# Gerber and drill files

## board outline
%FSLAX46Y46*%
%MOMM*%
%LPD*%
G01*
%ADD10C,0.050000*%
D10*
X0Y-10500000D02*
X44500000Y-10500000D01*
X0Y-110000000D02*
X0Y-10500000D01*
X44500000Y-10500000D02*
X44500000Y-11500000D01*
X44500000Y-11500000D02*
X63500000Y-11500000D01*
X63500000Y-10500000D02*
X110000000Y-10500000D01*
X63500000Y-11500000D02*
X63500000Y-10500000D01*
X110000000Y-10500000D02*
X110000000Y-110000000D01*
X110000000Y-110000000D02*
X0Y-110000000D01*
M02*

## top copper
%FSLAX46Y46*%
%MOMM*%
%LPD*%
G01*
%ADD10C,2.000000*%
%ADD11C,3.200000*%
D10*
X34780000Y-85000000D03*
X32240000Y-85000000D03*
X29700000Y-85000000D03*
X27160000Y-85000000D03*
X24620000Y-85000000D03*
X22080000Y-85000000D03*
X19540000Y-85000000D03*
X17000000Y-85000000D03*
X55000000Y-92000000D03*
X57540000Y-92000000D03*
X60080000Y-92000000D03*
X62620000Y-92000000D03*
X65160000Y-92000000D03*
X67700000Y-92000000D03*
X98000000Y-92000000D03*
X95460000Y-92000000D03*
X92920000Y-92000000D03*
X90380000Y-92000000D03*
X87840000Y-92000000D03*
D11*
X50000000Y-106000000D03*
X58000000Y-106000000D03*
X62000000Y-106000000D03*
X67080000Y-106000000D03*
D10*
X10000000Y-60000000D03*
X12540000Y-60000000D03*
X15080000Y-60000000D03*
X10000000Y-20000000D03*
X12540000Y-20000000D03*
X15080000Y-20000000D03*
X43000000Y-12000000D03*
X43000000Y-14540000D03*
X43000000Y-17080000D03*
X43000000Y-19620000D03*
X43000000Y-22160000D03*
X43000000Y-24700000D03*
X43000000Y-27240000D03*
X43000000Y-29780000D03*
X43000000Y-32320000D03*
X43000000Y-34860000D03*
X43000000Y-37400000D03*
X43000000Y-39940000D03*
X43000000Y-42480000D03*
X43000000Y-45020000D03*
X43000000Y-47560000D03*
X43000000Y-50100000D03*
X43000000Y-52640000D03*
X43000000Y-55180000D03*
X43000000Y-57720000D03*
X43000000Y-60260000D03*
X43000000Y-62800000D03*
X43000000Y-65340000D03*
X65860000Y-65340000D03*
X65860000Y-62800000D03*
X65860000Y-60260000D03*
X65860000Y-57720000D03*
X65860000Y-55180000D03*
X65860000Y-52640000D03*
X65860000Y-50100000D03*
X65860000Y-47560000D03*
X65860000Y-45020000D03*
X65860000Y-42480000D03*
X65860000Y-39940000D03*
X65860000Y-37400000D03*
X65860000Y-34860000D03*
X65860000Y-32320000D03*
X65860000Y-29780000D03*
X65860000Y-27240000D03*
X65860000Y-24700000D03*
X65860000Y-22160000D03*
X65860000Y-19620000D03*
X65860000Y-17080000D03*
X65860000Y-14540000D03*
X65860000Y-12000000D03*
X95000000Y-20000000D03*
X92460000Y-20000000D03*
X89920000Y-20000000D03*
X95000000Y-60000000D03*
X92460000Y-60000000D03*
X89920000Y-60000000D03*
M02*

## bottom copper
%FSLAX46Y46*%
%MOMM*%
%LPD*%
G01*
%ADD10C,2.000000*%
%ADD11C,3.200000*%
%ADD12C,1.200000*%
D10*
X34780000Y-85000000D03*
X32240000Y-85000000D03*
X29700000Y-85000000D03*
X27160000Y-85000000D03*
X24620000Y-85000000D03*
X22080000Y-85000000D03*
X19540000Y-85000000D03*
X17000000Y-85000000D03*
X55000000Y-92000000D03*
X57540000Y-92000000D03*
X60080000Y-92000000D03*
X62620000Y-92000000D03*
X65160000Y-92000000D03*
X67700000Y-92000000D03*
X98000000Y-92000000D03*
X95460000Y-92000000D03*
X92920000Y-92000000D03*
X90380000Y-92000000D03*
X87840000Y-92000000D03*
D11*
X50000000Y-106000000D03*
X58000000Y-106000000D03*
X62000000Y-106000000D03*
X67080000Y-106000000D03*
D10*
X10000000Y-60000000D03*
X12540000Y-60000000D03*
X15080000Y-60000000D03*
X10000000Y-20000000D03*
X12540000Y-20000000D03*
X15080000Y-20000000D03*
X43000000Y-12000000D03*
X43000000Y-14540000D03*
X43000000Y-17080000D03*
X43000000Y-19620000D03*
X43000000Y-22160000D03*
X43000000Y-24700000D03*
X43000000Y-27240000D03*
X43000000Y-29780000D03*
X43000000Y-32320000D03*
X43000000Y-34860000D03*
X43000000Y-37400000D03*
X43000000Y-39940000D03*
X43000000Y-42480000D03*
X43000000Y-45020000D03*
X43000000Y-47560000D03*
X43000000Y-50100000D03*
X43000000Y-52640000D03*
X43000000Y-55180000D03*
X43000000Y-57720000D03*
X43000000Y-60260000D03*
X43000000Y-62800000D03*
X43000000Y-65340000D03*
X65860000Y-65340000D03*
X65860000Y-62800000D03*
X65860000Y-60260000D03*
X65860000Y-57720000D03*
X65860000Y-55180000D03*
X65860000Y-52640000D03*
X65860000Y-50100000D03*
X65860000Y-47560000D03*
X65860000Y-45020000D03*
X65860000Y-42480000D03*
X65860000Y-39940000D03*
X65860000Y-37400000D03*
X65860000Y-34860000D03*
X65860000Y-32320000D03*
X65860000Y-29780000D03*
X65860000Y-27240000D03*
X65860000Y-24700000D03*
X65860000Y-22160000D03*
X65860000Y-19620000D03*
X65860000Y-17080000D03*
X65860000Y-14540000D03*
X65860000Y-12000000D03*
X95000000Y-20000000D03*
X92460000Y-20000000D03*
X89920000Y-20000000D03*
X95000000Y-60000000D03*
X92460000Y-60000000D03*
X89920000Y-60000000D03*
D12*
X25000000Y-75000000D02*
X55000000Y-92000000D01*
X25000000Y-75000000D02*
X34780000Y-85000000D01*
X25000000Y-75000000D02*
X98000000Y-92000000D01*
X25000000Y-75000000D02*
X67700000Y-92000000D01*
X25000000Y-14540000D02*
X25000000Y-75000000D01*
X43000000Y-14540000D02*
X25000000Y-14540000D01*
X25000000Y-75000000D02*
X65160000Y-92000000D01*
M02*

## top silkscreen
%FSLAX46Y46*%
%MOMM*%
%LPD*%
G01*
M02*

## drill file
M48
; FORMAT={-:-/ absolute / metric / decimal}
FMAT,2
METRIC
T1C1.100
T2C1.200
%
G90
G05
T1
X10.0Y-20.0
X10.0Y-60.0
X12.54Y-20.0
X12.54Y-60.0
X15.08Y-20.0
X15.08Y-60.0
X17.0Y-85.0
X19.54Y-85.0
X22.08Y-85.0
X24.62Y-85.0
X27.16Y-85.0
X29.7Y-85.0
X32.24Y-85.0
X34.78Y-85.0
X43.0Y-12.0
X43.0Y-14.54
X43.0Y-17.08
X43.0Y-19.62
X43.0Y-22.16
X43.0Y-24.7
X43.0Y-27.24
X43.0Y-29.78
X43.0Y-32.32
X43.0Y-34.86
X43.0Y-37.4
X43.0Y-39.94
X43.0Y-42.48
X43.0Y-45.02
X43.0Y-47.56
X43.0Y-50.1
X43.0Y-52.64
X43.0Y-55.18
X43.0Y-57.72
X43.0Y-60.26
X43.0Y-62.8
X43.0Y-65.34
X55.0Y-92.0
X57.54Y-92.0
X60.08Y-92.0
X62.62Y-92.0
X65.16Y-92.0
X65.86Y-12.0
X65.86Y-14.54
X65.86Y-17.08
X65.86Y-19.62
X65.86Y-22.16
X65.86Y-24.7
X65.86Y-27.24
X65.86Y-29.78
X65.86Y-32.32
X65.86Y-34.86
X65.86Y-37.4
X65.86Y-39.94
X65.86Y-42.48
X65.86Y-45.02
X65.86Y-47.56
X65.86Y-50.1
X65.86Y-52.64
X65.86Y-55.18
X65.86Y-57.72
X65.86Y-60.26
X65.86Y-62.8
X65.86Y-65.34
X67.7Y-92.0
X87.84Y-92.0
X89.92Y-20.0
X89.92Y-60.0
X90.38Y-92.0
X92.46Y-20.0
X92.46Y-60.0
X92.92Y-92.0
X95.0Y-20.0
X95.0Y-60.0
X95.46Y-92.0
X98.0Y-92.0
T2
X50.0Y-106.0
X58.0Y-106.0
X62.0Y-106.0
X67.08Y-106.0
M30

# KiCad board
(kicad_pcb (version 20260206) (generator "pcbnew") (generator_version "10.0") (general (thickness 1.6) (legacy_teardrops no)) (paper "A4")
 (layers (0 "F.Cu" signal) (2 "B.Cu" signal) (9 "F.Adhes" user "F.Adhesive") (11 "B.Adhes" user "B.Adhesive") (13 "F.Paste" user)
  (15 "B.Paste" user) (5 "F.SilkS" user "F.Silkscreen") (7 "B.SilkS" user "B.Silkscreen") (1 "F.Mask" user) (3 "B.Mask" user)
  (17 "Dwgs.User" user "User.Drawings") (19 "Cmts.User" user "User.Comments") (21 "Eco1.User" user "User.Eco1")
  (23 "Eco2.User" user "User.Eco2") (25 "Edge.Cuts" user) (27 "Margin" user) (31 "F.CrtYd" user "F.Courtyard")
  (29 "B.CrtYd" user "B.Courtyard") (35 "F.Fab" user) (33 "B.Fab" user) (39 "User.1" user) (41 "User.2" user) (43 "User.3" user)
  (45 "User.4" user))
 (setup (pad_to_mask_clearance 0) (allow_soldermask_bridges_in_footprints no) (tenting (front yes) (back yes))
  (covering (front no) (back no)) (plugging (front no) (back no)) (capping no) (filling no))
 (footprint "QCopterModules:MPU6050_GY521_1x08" (layer "F.Cu") (at 34.78 85 -90)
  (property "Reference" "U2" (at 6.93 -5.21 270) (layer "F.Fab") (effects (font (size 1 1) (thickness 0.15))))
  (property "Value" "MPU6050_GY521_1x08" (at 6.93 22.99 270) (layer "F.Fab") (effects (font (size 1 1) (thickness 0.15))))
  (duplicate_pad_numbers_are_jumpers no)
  (pad "1" thru_hole circle (at 0 0 270) (size 2 2) (drill 1.1) (layers "*.Cu" "*.Mask") (remove_unused_layers no) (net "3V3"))
  (pad "2" thru_hole circle (at 0 2.54 270) (size 2 2) (drill 1.1) (layers "*.Cu" "*.Mask") (remove_unused_layers no) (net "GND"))
  (pad "3" thru_hole circle (at 0 5.08 270) (size 2 2) (drill 1.1) (layers "*.Cu" "*.Mask") (remove_unused_layers no) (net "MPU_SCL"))
  (pad "4" thru_hole circle (at 0 7.62 270) (size 2 2) (drill 1.1) (layers "*.Cu" "*.Mask") (remove_unused_layers no) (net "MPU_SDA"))
  (pad "5" thru_hole circle (at 0 10.16 270) (size 2 2) (drill 1.1) (layers "*.Cu" "*.Mask") (remove_unused_layers no)
   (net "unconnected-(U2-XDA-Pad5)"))
  (pad "6" thru_hole circle (at 0 12.7 270) (size 2 2) (drill 1.1) (layers "*.Cu" "*.Mask") (remove_unused_layers no)
   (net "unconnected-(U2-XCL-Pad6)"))
  (pad "7" thru_hole circle (at 0 15.24 270) (size 2 2) (drill 1.1) (layers "*.Cu" "*.Mask") (remove_unused_layers no) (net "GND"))
  (pad "8" thru_hole circle (at 0 17.78 270) (size 2 2) (drill 1.1) (layers "*.Cu" "*.Mask") (remove_unused_layers no) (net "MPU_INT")))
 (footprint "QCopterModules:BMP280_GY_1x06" (layer "F.Cu") (at 55 92 90)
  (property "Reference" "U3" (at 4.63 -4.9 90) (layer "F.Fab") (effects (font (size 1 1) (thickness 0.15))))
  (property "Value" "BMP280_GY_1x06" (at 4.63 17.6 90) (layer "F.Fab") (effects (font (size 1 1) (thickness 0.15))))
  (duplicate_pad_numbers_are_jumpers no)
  (pad "1" thru_hole circle (at 0 0 90) (size 2 2) (drill 1.1) (layers "*.Cu" "*.Mask") (remove_unused_layers no) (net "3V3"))
  (pad "2" thru_hole circle (at 0 2.54 90) (size 2 2) (drill 1.1) (layers "*.Cu" "*.Mask") (remove_unused_layers no) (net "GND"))
  (pad "3" thru_hole circle (at 0 5.08 90) (size 2 2) (drill 1.1) (layers "*.Cu" "*.Mask") (remove_unused_layers no) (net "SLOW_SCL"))
  (pad "4" thru_hole circle (at 0 7.62 90) (size 2 2) (drill 1.1) (layers "*.Cu" "*.Mask") (remove_unused_layers no) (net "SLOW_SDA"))
  (pad "5" thru_hole circle (at 0 10.16 90) (size 2 2) (drill 1.1) (layers "*.Cu" "*.Mask") (remove_unused_layers no) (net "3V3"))
  (pad "6" thru_hole circle (at 0 12.7 90) (size 2 2) (drill 1.1) (layers "*.Cu" "*.Mask") (remove_unused_layers no) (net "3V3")))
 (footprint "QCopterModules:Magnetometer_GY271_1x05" (layer "F.Cu") (at 98 92 -90)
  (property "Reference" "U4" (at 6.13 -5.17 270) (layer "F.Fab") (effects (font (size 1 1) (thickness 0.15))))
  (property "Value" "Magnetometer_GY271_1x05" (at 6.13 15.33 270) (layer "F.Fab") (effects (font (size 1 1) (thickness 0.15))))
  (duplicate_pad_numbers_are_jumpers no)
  (pad "1" thru_hole circle (at 0 0 270) (size 2 2) (drill 1.1) (layers "*.Cu" "*.Mask") (remove_unused_layers no) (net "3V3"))
  (pad "2" thru_hole circle (at 0 2.54 270) (size 2 2) (drill 1.1) (layers "*.Cu" "*.Mask") (remove_unused_layers no) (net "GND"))
  (pad "3" thru_hole circle (at 0 5.08 270) (size 2 2) (drill 1.1) (layers "*.Cu" "*.Mask") (remove_unused_layers no) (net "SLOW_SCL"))
  (pad "4" thru_hole circle (at 0 7.62 270) (size 2 2) (drill 1.1) (layers "*.Cu" "*.Mask") (remove_unused_layers no) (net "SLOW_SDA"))
  (pad "5" thru_hole circle (at 0 10.16 270) (size 2 2) (drill 1.1) (layers "*.Cu" "*.Mask") (remove_unused_layers no) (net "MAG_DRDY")))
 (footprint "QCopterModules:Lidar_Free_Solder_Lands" (layer "F.Cu") (at 50 106)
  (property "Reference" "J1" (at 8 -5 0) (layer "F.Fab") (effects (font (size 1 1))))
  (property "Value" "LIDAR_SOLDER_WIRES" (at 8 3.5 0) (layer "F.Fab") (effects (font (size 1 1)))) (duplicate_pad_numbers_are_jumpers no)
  (pad "1" thru_hole circle (at 0 0) (size 3.2 3.2) (drill 1.2) (layers "*.Cu" "*.Mask") (remove_unused_layers no) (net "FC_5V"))
  (pad "2" thru_hole circle (at 8 0) (size 3.2 3.2) (drill 1.2) (layers "*.Cu" "*.Mask") (remove_unused_layers no) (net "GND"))
  (pad "3" thru_hole circle (at 12 0) (size 3.2 3.2) (drill 1.2) (layers "*.Cu" "*.Mask") (remove_unused_layers no) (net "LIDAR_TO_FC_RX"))
  (pad "4" thru_hole circle (at 17.08 0) (size 3.2 3.2) (drill 1.2) (layers "*.Cu" "*.Mask") (remove_unused_layers no)
   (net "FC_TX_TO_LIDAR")))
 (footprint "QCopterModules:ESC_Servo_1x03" (layer "F.Cu") (at 10 60 90)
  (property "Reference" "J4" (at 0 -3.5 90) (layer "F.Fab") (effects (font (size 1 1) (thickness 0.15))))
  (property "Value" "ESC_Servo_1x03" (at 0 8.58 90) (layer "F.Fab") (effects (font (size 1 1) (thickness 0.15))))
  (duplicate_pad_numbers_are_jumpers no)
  (pad "1" thru_hole circle (at 0 0 90) (size 2 2) (drill 1.1) (layers "*.Cu" "*.Mask") (remove_unused_layers no) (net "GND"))
  (pad "2" thru_hole circle (at 0 2.54 90) (size 2 2) (drill 1.1) (layers "*.Cu" "*.Mask") (remove_unused_layers no) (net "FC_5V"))
  (pad "3" thru_hole circle (at 0 5.08 90) (size 2 2) (drill 1.1) (layers "*.Cu" "*.Mask") (remove_unused_layers no) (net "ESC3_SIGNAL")))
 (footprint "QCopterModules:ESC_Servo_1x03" (layer "F.Cu") (at 10 20 90)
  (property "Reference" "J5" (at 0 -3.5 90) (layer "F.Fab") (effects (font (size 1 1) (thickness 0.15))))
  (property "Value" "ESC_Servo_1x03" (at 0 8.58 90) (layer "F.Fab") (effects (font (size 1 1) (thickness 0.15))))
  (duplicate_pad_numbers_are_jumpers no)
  (pad "1" thru_hole circle (at 0 0 90) (size 2 2) (drill 1.1) (layers "*.Cu" "*.Mask") (remove_unused_layers no) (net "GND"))
  (pad "2" thru_hole circle (at 0 2.54 90) (size 2 2) (drill 1.1) (layers "*.Cu" "*.Mask") (remove_unused_layers no)
   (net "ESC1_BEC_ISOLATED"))
  (pad "3" thru_hole circle (at 0 5.08 90) (size 2 2) (drill 1.1) (layers "*.Cu" "*.Mask") (remove_unused_layers no) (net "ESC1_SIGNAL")))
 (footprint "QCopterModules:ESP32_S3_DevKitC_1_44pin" (layer "F.Cu") (at 43 12)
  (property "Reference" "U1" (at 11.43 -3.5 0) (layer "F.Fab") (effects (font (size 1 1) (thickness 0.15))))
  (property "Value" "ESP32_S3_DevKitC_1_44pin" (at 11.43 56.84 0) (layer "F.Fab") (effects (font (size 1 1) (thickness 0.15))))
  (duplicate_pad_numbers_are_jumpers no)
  (pad "1" thru_hole circle (at 0 0) (size 2 2) (drill 1.1) (layers "*.Cu" "*.Mask") (remove_unused_layers no))
  (pad "2" thru_hole circle (at 0 2.54) (size 2 2) (drill 1.1) (layers "*.Cu" "*.Mask") (remove_unused_layers no) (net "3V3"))
  (pad "3" thru_hole circle (at 0 5.08) (size 2 2) (drill 1.1) (layers "*.Cu" "*.Mask") (remove_unused_layers no)
   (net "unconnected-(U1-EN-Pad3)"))
  (pad "4" thru_hole circle (at 0 7.62) (size 2 2) (drill 1.1) (layers "*.Cu" "*.Mask") (remove_unused_layers no) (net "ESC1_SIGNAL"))
  (pad "5" thru_hole circle (at 0 10.16) (size 2 2) (drill 1.1) (layers "*.Cu" "*.Mask") (remove_unused_layers no)
   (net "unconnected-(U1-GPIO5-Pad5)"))
  (pad "6" thru_hole circle (at 0 12.7) (size 2 2) (drill 1.1) (layers "*.Cu" "*.Mask") (remove_unused_layers no)
   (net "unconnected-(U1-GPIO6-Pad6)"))
  (pad "7" thru_hole circle (at 0 15.24) (size 2 2) (drill 1.1) (layers "*.Cu" "*.Mask") (remove_unused_layers no)
   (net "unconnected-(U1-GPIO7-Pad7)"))
  (pad "8" thru_hole circle (at 0 17.78) (size 2 2) (drill 1.1) (layers "*.Cu" "*.Mask") (remove_unused_layers no) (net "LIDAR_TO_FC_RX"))
  (pad "9" thru_hole circle (at 0 20.32) (size 2 2) (drill 1.1) (layers "*.Cu" "*.Mask") (remove_unused_layers no) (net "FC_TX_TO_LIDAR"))
  (pad "10" thru_hole circle (at 0 22.86) (size 2 2) (drill 1.1) (layers "*.Cu" "*.Mask") (remove_unused_layers no)
   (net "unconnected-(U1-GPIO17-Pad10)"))
  (pad "11" thru_hole circle (at 0 25.4) (size 2 2) (drill 1.1) (layers "*.Cu" "*.Mask") (remove_unused_layers no) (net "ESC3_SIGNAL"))
  (pad "12" thru_hole circle (at 0 27.94) (size 2 2) (drill 1.1) (layers "*.Cu" "*.Mask") (remove_unused_layers no)
   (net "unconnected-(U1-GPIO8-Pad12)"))
  (pad "13" thru_hole circle (at 0 30.48) (size 2 2) (drill 1.1) (layers "*.Cu" "*.Mask") (remove_unused_layers no)
   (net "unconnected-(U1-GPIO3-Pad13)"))
  (pad "14" thru_hole circle (at 0 33.02) (size 2 2) (drill 1.1) (layers "*.Cu" "*.Mask") (remove_unused_layers no)
   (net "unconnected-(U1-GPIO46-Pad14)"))
  (pad "15" thru_hole circle (at 0 35.56) (size 2 2) (drill 1.1) (layers "*.Cu" "*.Mask") (remove_unused_layers no)
   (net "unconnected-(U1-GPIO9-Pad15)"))
  (pad "16" thru_hole circle (at 0 38.1) (size 2 2) (drill 1.1) (layers "*.Cu" "*.Mask") (remove_unused_layers no)
   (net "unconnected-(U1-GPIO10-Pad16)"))
  (pad "17" thru_hole circle (at 0 40.64) (size 2 2) (drill 1.1) (layers "*.Cu" "*.Mask") (remove_unused_layers no)
   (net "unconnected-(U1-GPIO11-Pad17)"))
  (pad "18" thru_hole circle (at 0 43.18) (size 2 2) (drill 1.1) (layers "*.Cu" "*.Mask") (remove_unused_layers no) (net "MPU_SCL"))
  (pad "19" thru_hole circle (at 0 45.72) (size 2 2) (drill 1.1) (layers "*.Cu" "*.Mask") (remove_unused_layers no) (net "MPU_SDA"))
  (pad "20" thru_hole circle (at 0 48.26) (size 2 2) (drill 1.1) (layers "*.Cu" "*.Mask") (remove_unused_layers no) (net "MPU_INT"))
  (pad "21" thru_hole circle (at 0 50.8) (size 2 2) (drill 1.1) (layers "*.Cu" "*.Mask") (remove_unused_layers no) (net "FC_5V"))
  (pad "22" thru_hole circle (at 0 53.34) (size 2 2) (drill 1.1) (layers "*.Cu" "*.Mask") (remove_unused_layers no) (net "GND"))
  (pad "23" thru_hole circle (at 22.86 53.34) (size 2 2) (drill 1.1) (layers "*.Cu" "*.Mask") (remove_unused_layers no) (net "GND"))
  (pad "24" thru_hole circle (at 22.86 50.8) (size 2 2) (drill 1.1) (layers "*.Cu" "*.Mask") (remove_unused_layers no) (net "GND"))
  (pad "25" thru_hole circle (at 22.86 48.26) (size 2 2) (drill 1.1) (layers "*.Cu" "*.Mask") (remove_unused_layers no)
   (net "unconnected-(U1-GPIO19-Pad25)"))
  (pad "26" thru_hole circle (at 22.86 45.72) (size 2 2) (drill 1.1) (layers "*.Cu" "*.Mask") (remove_unused_layers no)
   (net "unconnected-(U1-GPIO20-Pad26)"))
  (pad "27" thru_hole circle (at 22.86 43.18) (size 2 2) (drill 1.1) (layers "*.Cu" "*.Mask") (remove_unused_layers no) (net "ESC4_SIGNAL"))
  (pad "28" thru_hole circle (at 22.86 40.64) (size 2 2) (drill 1.1) (layers "*.Cu" "*.Mask") (remove_unused_layers no)
   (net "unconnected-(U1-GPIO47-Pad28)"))
  (pad "29" thru_hole circle (at 22.86 38.1) (size 2 2) (drill 1.1) (layers "*.Cu" "*.Mask") (remove_unused_layers no)
   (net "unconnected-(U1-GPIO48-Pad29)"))
  (pad "30" thru_hole circle (at 22.86 35.56) (size 2 2) (drill 1.1) (layers "*.Cu" "*.Mask") (remove_unused_layers no)
   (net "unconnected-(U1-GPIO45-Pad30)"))
  (pad "31" thru_hole circle (at 22.86 33.02) (size 2 2) (drill 1.1) (layers "*.Cu" "*.Mask") (remove_unused_layers no)
   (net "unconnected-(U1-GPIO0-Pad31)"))
  (pad "32" thru_hole circle (at 22.86 30.48) (size 2 2) (drill 1.1) (layers "*.Cu" "*.Mask") (remove_unused_layers no)
   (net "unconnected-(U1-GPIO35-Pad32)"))
  (pad "33" thru_hole circle (at 22.86 27.94) (size 2 2) (drill 1.1) (layers "*.Cu" "*.Mask") (remove_unused_layers no)
   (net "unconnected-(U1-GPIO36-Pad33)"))
  (pad "34" thru_hole circle (at 22.86 25.4) (size 2 2) (drill 1.1) (layers "*.Cu" "*.Mask") (remove_unused_layers no)
   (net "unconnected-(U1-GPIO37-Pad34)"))
  (pad "35" thru_hole circle (at 22.86 22.86) (size 2 2) (drill 1.1) (layers "*.Cu" "*.Mask") (remove_unused_layers no)
   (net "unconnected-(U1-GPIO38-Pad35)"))
  (pad "36" thru_hole circle (at 22.86 20.32) (size 2 2) (drill 1.1) (layers "*.Cu" "*.Mask") (remove_unused_layers no) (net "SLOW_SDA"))
  (pad "37" thru_hole circle (at 22.86 17.78) (size 2 2) (drill 1.1) (layers "*.Cu" "*.Mask") (remove_unused_layers no) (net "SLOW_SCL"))
  (pad "38" thru_hole circle (at 22.86 15.24) (size 2 2) (drill 1.1) (layers "*.Cu" "*.Mask") (remove_unused_layers no) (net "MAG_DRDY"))
  (pad "39" thru_hole circle (at 22.86 12.7) (size 2 2) (drill 1.1) (layers "*.Cu" "*.Mask") (remove_unused_layers no)
   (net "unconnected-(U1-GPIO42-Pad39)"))
  (pad "40" thru_hole circle (at 22.86 10.16) (size 2 2) (drill 1.1) (layers "*.Cu" "*.Mask") (remove_unused_layers no) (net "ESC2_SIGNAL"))
  (pad "41" thru_hole circle (at 22.86 7.62) (size 2 2) (drill 1.1) (layers "*.Cu" "*.Mask") (remove_unused_layers no)
   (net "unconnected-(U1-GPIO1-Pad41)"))
  (pad "42" thru_hole circle (at 22.86 5.08) (size 2 2) (drill 1.1) (layers "*.Cu" "*.Mask") (remove_unused_layers no)
   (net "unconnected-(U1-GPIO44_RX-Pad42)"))
  (pad "43" thru_hole circle (at 22.86 2.54) (size 2 2) (drill 1.1) (layers "*.Cu" "*.Mask") (remove_unused_layers no)
   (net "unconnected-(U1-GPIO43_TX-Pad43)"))
  (pad "44" thru_hole circle (at 22.86 0) (size 2 2) (drill 1.1) (layers "*.Cu" "*.Mask") (remove_unused_layers no) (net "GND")))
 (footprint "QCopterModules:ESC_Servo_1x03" (layer "F.Cu") (at 95 20 -90)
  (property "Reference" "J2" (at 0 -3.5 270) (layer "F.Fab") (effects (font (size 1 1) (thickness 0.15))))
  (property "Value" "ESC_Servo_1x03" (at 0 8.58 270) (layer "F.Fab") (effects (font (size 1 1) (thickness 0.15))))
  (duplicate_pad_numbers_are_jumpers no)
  (pad "1" thru_hole circle (at 0 0 270) (size 2 2) (drill 1.1) (layers "*.Cu" "*.Mask") (remove_unused_layers no) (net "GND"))
  (pad "2" thru_hole circle (at 0 2.54 270) (size 2 2) (drill 1.1) (layers "*.Cu" "*.Mask") (remove_unused_layers no)
   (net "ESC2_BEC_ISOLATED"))
  (pad "3" thru_hole circle (at 0 5.08 270) (size 2 2) (drill 1.1) (layers "*.Cu" "*.Mask") (remove_unused_layers no) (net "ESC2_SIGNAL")))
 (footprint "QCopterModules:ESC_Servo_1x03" (layer "F.Cu") (at 95 60 -90)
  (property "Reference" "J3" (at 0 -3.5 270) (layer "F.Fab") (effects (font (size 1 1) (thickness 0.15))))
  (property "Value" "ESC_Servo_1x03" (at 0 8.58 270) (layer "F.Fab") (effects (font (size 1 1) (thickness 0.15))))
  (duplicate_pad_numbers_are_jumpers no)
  (pad "1" thru_hole circle (at 0 0 270) (size 2 2) (drill 1.1) (layers "*.Cu" "*.Mask") (remove_unused_layers no) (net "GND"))
  (pad "2" thru_hole circle (at 0 2.54 270) (size 2 2) (drill 1.1) (layers "*.Cu" "*.Mask") (remove_unused_layers no)
   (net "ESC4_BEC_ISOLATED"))
  (pad "3" thru_hole circle (at 0 5.08 270) (size 2 2) (drill 1.1) (layers "*.Cu" "*.Mask") (remove_unused_layers no) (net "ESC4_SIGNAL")))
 (gr_line (start 0 10.5) (end 44.5 10.5) (stroke (width 0.05) (type default)) (layer "Edge.Cuts"))
 (gr_line (start 0 110) (end 0 10.5) (stroke (width 0.05) (type default)) (layer "Edge.Cuts"))
 (gr_line (start 44.5 10.5) (end 44.5 11.5) (stroke (width 0.05) (type default)) (layer "Edge.Cuts"))
 (gr_line (start 44.5 11.5) (end 63.5 11.5) (stroke (width 0.05) (type default)) (layer "Edge.Cuts"))
 (gr_line (start 63.5 10.5) (end 110 10.5) (stroke (width 0.05) (type default)) (layer "Edge.Cuts"))
 (gr_line (start 63.5 11.5) (end 63.5 10.5) (stroke (width 0.05) (type default)) (layer "Edge.Cuts"))
 (gr_line (start 110 10.5) (end 110 110) (stroke (width 0.05) (type default)) (layer "Edge.Cuts"))
 (gr_line (start 110 110) (end 0 110) (stroke (width 0.05) (type default)) (layer "Edge.Cuts"))
 (segment (start 25 75) (end 55 92) (width 1.2) (layer "B.Cu") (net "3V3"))
 (segment (start 25 75) (end 34.78 85) (width 1.2) (layer "B.Cu") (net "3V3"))
 (segment (start 25 75) (end 98 92) (width 1.2) (layer "B.Cu") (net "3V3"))
 (segment (start 25 75) (end 67.7 92) (width 1.2) (layer "B.Cu") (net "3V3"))
 (segment (start 25 14.54) (end 25 75) (width 1.2) (layer "B.Cu") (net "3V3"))
 (segment (start 43 14.54) (end 25 14.54) (width 1.2) (layer "B.Cu") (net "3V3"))
 (segment (start 25 75) (end 65.16 92) (width 1.2) (layer "B.Cu") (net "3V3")))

